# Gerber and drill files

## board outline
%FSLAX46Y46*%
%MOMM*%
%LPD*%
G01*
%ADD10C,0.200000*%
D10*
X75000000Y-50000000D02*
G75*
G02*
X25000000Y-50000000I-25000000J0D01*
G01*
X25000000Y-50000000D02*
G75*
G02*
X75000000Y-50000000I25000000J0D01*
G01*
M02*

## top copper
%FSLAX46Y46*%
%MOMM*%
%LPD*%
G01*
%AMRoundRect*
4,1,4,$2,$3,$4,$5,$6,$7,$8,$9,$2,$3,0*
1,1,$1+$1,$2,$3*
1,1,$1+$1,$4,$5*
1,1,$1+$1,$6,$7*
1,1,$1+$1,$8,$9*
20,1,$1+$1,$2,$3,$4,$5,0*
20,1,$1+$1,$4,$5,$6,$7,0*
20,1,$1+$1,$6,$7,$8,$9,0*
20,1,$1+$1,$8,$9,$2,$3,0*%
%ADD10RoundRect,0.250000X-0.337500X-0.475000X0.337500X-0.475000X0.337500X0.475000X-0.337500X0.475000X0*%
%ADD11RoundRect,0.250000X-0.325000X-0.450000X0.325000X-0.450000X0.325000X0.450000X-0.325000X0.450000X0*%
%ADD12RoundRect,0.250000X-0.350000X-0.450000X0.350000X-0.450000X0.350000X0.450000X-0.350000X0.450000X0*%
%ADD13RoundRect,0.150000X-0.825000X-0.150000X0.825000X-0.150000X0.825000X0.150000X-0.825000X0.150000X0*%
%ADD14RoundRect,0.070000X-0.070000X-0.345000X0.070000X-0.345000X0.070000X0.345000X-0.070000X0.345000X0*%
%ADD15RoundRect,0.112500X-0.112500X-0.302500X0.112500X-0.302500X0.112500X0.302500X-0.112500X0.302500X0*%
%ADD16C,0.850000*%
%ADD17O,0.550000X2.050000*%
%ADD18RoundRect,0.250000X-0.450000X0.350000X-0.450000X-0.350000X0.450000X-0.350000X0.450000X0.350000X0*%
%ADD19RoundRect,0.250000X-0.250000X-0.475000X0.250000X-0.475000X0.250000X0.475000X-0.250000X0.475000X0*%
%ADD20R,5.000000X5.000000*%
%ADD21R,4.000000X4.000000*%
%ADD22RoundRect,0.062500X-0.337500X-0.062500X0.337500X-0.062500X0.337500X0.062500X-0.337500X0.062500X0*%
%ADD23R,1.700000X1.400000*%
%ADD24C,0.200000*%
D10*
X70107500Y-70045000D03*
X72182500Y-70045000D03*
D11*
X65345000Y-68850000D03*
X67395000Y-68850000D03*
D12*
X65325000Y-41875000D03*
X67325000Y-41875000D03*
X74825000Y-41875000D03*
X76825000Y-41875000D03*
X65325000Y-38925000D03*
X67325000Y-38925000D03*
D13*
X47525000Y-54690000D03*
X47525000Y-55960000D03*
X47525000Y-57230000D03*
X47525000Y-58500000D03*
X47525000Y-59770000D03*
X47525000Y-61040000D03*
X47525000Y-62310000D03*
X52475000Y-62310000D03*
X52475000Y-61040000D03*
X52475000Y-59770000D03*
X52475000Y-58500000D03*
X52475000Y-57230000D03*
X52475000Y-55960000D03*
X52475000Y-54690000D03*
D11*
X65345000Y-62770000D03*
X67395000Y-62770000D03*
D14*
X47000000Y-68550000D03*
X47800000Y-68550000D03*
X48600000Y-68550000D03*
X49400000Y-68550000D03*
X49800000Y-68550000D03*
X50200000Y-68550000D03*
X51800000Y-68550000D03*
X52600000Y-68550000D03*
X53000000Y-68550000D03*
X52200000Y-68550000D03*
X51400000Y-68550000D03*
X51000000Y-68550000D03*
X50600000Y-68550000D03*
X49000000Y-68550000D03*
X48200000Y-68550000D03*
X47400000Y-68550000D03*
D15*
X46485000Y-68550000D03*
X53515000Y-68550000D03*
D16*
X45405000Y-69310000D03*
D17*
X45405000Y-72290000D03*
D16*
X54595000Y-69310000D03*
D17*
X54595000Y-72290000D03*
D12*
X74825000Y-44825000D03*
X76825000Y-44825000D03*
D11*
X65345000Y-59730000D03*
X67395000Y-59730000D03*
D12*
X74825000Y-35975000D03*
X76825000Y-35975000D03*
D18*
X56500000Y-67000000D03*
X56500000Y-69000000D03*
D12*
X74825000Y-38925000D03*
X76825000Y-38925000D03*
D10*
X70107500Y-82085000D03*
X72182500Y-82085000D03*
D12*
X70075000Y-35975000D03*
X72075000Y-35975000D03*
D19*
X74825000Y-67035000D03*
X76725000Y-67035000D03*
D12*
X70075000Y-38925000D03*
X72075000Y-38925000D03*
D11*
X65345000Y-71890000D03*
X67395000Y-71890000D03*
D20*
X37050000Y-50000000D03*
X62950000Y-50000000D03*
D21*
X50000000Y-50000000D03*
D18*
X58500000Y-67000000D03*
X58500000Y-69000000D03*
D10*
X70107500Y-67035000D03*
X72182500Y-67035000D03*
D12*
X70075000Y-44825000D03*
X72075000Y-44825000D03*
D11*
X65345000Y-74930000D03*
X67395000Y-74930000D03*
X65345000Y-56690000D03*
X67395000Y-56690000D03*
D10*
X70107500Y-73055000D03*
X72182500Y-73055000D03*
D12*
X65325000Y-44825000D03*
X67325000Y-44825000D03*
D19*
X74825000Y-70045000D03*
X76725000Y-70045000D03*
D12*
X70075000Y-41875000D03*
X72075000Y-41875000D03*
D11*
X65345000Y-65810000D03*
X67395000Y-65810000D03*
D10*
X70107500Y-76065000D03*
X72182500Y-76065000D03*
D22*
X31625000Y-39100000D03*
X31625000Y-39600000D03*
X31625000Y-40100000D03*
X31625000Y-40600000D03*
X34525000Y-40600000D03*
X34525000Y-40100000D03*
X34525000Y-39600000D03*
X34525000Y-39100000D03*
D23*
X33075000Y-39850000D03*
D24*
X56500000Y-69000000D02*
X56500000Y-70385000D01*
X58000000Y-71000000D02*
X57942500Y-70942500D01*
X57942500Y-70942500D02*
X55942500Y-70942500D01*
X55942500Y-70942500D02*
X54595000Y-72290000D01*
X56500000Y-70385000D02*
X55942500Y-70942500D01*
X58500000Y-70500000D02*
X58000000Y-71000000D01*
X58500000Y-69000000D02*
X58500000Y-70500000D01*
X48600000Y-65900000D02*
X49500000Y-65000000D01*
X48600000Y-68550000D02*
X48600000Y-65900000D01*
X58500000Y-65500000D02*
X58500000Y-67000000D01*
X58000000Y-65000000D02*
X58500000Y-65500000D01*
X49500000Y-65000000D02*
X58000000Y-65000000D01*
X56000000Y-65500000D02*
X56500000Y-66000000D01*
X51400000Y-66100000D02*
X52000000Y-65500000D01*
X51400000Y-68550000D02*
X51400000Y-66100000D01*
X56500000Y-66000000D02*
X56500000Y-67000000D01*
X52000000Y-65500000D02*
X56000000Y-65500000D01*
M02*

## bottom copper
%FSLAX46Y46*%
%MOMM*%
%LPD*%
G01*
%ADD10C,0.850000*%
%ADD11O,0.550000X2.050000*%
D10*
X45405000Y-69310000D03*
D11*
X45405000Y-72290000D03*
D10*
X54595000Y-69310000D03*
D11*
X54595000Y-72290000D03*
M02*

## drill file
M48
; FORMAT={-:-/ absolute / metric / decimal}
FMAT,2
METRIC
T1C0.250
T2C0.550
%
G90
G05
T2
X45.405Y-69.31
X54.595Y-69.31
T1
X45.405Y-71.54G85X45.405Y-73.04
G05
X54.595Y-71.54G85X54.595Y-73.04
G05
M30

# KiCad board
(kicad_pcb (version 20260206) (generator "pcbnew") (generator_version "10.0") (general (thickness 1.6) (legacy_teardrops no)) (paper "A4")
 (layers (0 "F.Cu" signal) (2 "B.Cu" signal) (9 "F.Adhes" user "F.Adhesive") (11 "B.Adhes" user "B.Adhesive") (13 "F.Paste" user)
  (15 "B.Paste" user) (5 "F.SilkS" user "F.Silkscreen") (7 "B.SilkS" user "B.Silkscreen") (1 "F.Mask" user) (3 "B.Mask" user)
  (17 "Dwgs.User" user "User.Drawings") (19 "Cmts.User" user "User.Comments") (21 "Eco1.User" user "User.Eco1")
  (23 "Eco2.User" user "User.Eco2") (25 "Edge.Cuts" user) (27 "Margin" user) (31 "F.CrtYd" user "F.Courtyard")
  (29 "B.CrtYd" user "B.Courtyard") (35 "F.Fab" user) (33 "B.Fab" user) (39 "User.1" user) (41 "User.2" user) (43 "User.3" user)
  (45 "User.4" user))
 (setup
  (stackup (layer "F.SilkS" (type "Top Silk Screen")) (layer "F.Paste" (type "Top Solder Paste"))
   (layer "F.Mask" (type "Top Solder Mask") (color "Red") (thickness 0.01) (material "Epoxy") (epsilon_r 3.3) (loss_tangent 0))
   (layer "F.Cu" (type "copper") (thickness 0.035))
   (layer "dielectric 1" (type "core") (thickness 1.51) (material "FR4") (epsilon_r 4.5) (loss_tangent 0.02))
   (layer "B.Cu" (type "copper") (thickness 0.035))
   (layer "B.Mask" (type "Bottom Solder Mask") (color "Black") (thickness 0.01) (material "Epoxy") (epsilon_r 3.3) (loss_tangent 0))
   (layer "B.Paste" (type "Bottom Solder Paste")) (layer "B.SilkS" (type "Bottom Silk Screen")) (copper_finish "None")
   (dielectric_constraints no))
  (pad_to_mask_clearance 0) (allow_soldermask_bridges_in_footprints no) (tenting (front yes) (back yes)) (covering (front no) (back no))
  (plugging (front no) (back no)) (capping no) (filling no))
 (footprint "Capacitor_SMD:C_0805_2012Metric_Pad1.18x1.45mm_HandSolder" (layer "F.Cu") (at 71.145 70.045)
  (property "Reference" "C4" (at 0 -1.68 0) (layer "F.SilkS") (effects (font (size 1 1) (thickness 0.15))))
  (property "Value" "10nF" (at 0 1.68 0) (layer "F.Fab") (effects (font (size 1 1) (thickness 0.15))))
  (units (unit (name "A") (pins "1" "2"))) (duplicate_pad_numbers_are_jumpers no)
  (pad "1" smd roundrect (at -1.0375 0) (size 1.175 1.45) (layers "F.Cu" "F.Mask" "F.Paste") (roundrect_rratio 0.212766) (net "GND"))
  (pad "2" smd roundrect (at 1.0375 0) (size 1.175 1.45) (layers "F.Cu" "F.Mask" "F.Paste") (roundrect_rratio 0.212766)
   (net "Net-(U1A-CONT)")))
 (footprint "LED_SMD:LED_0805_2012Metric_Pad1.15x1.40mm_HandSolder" (layer "F.Cu") (at 66.37 68.85)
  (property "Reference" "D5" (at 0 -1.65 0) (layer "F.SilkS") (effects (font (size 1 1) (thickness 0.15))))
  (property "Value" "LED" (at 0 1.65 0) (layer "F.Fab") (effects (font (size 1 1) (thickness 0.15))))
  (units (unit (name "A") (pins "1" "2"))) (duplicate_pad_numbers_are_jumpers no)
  (pad "1" smd roundrect (at -1.025 0) (size 1.15 1.4) (layers "F.Cu" "F.Mask" "F.Paste") (roundrect_rratio 0.217391) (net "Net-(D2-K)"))
  (pad "2" smd roundrect (at 1.025 0) (size 1.15 1.4) (layers "F.Cu" "F.Mask" "F.Paste") (roundrect_rratio 0.217391) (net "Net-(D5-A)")))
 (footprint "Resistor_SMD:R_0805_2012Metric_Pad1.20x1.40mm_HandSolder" (layer "F.Cu") (at 66.325 41.875)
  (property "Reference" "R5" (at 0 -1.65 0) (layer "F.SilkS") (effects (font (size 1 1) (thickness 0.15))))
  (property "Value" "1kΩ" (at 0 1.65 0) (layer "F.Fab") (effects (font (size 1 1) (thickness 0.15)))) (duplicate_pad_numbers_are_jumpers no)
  (pad "1" smd roundrect (at -1 0) (size 1.2 1.4) (layers "F.Cu" "F.Mask" "F.Paste") (roundrect_rratio 0.208333) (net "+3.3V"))
  (pad "2" smd roundrect (at 1 0) (size 1.2 1.4) (layers "F.Cu" "F.Mask" "F.Paste") (roundrect_rratio 0.208333) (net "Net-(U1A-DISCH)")))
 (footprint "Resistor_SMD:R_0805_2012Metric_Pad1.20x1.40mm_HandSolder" (layer "F.Cu") (at 75.825 41.875)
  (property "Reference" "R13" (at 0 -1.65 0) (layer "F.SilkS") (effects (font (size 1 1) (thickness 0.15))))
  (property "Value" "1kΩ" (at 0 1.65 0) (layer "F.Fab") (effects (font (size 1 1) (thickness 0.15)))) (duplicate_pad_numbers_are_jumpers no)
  (pad "1" smd roundrect (at -1 0) (size 1.2 1.4) (layers "F.Cu" "F.Mask" "F.Paste") (roundrect_rratio 0.208333) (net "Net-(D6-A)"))
  (pad "2" smd roundrect (at 1 0) (size 1.2 1.4) (layers "F.Cu" "F.Mask" "F.Paste") (roundrect_rratio 0.208333) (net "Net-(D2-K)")))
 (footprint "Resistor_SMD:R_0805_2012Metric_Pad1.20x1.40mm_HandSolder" (layer "F.Cu") (at 66.325 38.925)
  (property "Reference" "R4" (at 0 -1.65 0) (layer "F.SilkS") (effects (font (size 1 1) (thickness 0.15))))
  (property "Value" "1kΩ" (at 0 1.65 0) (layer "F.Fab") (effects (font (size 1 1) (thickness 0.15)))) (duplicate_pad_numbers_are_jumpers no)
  (pad "1" smd roundrect (at -1 0) (size 1.2 1.4) (layers "F.Cu" "F.Mask" "F.Paste") (roundrect_rratio 0.208333) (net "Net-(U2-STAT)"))
  (pad "2" smd roundrect (at 1 0) (size 1.2 1.4) (layers "F.Cu" "F.Mask" "F.Paste") (roundrect_rratio 0.208333) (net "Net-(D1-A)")))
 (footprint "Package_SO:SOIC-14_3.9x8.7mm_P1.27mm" (layer "F.Cu") (at 50 58.5)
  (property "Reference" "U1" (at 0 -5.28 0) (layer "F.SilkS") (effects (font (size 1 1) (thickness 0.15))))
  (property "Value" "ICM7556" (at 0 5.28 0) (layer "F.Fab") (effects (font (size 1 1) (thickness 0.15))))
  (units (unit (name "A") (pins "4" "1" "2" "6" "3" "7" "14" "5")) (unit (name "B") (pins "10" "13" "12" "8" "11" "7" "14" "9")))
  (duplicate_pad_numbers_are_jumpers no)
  (pad "1" smd roundrect (at -2.475 -3.81) (size 1.95 0.6) (layers "F.Cu" "F.Mask" "F.Paste") (roundrect_rratio 0.25)
   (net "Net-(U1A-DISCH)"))
  (pad "2" smd roundrect (at -2.475 -2.54) (size 1.95 0.6) (layers "F.Cu" "F.Mask" "F.Paste") (roundrect_rratio 0.25)
   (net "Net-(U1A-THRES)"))
  (pad "3" smd roundrect (at -2.475 -1.27) (size 1.95 0.6) (layers "F.Cu" "F.Mask" "F.Paste") (roundrect_rratio 0.25) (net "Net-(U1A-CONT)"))
  (pad "4" smd roundrect (at -2.475 0) (size 1.95 0.6) (layers "F.Cu" "F.Mask" "F.Paste") (roundrect_rratio 0.25) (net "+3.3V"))
  (pad "5" smd roundrect (at -2.475 1.27) (size 1.95 0.6) (layers "F.Cu" "F.Mask" "F.Paste") (roundrect_rratio 0.25) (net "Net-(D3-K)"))
  (pad "6" smd roundrect (at -2.475 2.54) (size 1.95 0.6) (layers "F.Cu" "F.Mask" "F.Paste") (roundrect_rratio 0.25) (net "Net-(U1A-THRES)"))
  (pad "7" smd roundrect (at -2.475 3.81) (size 1.95 0.6) (layers "F.Cu" "F.Mask" "F.Paste") (roundrect_rratio 0.25) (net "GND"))
  (pad "8" smd roundrect (at 2.475 3.81) (size 1.95 0.6) (layers "F.Cu" "F.Mask" "F.Paste") (roundrect_rratio 0.25) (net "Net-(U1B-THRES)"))
  (pad "9" smd roundrect (at 2.475 2.54) (size 1.95 0.6) (layers "F.Cu" "F.Mask" "F.Paste") (roundrect_rratio 0.25) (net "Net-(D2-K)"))
  (pad "10" smd roundrect (at 2.475 1.27) (size 1.95 0.6) (layers "F.Cu" "F.Mask" "F.Paste") (roundrect_rratio 0.25) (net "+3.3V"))
  (pad "11" smd roundrect (at 2.475 0) (size 1.95 0.6) (layers "F.Cu" "F.Mask" "F.Paste") (roundrect_rratio 0.25) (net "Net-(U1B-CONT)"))
  (pad "12" smd roundrect (at 2.475 -1.27) (size 1.95 0.6) (layers "F.Cu" "F.Mask" "F.Paste") (roundrect_rratio 0.25)
   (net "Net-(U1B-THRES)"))
  (pad "13" smd roundrect (at 2.475 -2.54) (size 1.95 0.6) (layers "F.Cu" "F.Mask" "F.Paste") (roundrect_rratio 0.25)
   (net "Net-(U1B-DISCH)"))
  (pad "14" smd roundrect (at 2.475 -3.81) (size 1.95 0.6) (layers "F.Cu" "F.Mask" "F.Paste") (roundrect_rratio 0.25) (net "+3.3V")))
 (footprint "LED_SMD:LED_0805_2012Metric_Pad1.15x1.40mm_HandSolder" (layer "F.Cu") (at 66.37 62.77)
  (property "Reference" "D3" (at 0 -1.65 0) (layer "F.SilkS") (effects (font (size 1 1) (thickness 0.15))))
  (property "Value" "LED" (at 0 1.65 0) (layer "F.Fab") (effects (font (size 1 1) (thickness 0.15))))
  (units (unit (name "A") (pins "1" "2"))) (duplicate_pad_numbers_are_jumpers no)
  (pad "1" smd roundrect (at -1.025 0) (size 1.15 1.4) (layers "F.Cu" "F.Mask" "F.Paste") (roundrect_rratio 0.217391) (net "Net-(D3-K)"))
  (pad "2" smd roundrect (at 1.025 0) (size 1.15 1.4) (layers "F.Cu" "F.Mask" "F.Paste") (roundrect_rratio 0.217391) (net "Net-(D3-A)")))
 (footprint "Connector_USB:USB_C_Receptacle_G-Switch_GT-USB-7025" (layer "F.Cu") (at 50 72)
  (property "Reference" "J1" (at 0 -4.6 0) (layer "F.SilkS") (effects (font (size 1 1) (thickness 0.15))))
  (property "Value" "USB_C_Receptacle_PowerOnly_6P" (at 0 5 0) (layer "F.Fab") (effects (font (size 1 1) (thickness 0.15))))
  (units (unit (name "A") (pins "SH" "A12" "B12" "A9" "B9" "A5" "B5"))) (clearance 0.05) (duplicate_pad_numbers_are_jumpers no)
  (pad "A1" smd roundrect (at -3 -3.45) (size 0.28 0.83) (layers "F.Cu" "F.Mask" "F.Paste") (roundrect_rratio 0.25))
  (pad "A4" smd roundrect (at -2.2 -3.45) (size 0.28 0.83) (layers "F.Cu" "F.Mask" "F.Paste") (roundrect_rratio 0.25))
  (pad "A5" smd roundrect (at -1.4 -3.45) (size 0.28 0.83) (layers "F.Cu" "F.Mask" "F.Paste") (roundrect_rratio 0.25) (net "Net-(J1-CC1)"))
  (pad "A6" smd roundrect (at -0.6 -3.45) (size 0.28 0.83) (layers "F.Cu" "F.Mask" "F.Paste") (roundrect_rratio 0.25))
  (pad "A7" smd roundrect (at -0.2 -3.45) (size 0.28 0.83) (layers "F.Cu" "F.Mask" "F.Paste") (roundrect_rratio 0.25))
  (pad "A8" smd roundrect (at 0.2 -3.45) (size 0.28 0.83) (layers "F.Cu" "F.Mask" "F.Paste") (roundrect_rratio 0.25))
  (pad "A9" smd roundrect (at 1.8 -3.45) (size 0.28 0.83) (layers "F.Cu" "F.Mask" "F.Paste") (roundrect_rratio 0.25) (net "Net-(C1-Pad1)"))
  (pad "A12" smd roundrect (at 2.6 -3.45) (size 0.28 0.83) (layers "F.Cu" "F.Mask" "F.Paste") (roundrect_rratio 0.25) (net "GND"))
  (pad "B1" smd roundrect (at 3 -3.45) (size 0.28 0.83) (layers "F.Cu" "F.Mask" "F.Paste") (roundrect_rratio 0.25))
  (pad "B4" smd roundrect (at 2.2 -3.45) (size 0.28 0.83) (layers "F.Cu" "F.Mask" "F.Paste") (roundrect_rratio 0.25))
  (pad "B5" smd roundrect (at 1.4 -3.45) (size 0.28 0.83) (layers "F.Cu" "F.Mask" "F.Paste") (roundrect_rratio 0.25) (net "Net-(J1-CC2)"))
  (pad "B6" smd roundrect (at 1 -3.45) (size 0.28 0.83) (layers "F.Cu" "F.Mask" "F.Paste") (roundrect_rratio 0.25))
  (pad "B7" smd roundrect (at 0.6 -3.45) (size 0.28 0.83) (layers "F.Cu" "F.Mask" "F.Paste") (roundrect_rratio 0.25))
  (pad "B8" smd roundrect (at -1 -3.45) (size 0.28 0.83) (layers "F.Cu" "F.Mask" "F.Paste") (roundrect_rratio 0.25))
  (pad "B9" smd roundrect (at -1.8 -3.45) (size 0.28 0.83) (layers "F.Cu" "F.Mask" "F.Paste") (roundrect_rratio 0.25) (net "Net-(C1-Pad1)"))
  (pad "B12" smd roundrect (at -2.6 -3.45) (size 0.28 0.83) (layers "F.Cu" "F.Mask" "F.Paste") (roundrect_rratio 0.25) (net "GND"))
  (pad "GND" smd roundrect (at -3.515 -3.45) (size 0.45 0.83) (layers "F.Cu" "F.Mask" "F.Paste") (roundrect_rratio 0.25))
  (pad "GND" smd roundrect (at 3.515 -3.45) (size 0.45 0.83) (layers "F.Cu" "F.Mask" "F.Paste") (roundrect_rratio 0.25))
  (pad "SH" thru_hole circle (at -4.595 -2.69) (size 0.85 0.85) (drill 0.55) (layers "*.Cu" "*.Mask") (remove_unused_layers no) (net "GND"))
  (pad "SH" thru_hole oval (at -4.595 0.29) (size 0.55 2.05) (drill oval 0.25 1.75) (layers "*.Cu" "*.Mask") (remove_unused_layers no)
   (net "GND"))
  (pad "SH" thru_hole circle (at 4.595 -2.69) (size 0.85 0.85) (drill 0.55) (layers "*.Cu" "*.Mask") (remove_unused_layers no) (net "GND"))
  (pad "SH" thru_hole oval (at 4.595 0.29) (size 0.55 2.05) (drill oval 0.25 1.75) (layers "*.Cu" "*.Mask") (remove_unused_layers no)
   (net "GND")))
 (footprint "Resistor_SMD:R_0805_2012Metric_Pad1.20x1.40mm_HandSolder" (layer "F.Cu") (at 75.825 44.825)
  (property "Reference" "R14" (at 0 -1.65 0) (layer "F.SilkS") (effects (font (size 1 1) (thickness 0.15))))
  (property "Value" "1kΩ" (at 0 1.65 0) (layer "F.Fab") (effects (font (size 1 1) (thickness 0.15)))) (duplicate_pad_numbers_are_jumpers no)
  (pad "1" smd roundrect (at -1 0) (size 1.2 1.4) (layers "F.Cu" "F.Mask" "F.Paste") (roundrect_rratio 0.208333) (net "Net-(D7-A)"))
  (pad "2" smd roundrect (at 1 0) (size 1.2 1.4) (layers "F.Cu" "F.Mask" "F.Paste") (roundrect_rratio 0.208333) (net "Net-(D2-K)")))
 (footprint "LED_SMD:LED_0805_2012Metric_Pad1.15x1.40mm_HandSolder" (layer "F.Cu") (at 66.37 59.73)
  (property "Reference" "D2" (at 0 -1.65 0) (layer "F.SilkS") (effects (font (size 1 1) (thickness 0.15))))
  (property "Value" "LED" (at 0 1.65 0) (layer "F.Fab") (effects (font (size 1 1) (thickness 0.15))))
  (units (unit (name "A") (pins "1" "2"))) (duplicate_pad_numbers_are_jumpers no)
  (pad "1" smd roundrect (at -1.025 0) (size 1.15 1.4) (layers "F.Cu" "F.Mask" "F.Paste") (roundrect_rratio 0.217391) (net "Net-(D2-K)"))
  (pad "2" smd roundrect (at 1.025 0) (size 1.15 1.4) (layers "F.Cu" "F.Mask" "F.Paste") (roundrect_rratio 0.217391) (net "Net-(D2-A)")))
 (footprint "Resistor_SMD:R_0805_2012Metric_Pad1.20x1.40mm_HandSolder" (layer "F.Cu") (at 75.825 35.975)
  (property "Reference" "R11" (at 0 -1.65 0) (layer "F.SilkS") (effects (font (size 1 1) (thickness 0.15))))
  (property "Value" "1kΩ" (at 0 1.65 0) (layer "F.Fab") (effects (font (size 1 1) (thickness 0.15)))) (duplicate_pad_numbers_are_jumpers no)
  (pad "1" smd roundrect (at -1 0) (size 1.2 1.4) (layers "F.Cu" "F.Mask" "F.Paste") (roundrect_rratio 0.208333) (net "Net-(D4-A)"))
  (pad "2" smd roundrect (at 1 0) (size 1.2 1.4) (layers "F.Cu" "F.Mask" "F.Paste") (roundrect_rratio 0.208333) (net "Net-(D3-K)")))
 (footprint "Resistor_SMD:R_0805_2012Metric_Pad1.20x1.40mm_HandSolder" (layer "F.Cu") (at 56.5 68 -90)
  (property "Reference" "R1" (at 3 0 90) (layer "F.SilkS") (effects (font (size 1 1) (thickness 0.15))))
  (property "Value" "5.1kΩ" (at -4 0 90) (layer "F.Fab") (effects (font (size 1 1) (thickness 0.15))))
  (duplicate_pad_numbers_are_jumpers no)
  (pad "1" smd roundrect (at -1 0 270) (size 1.2 1.4) (layers "F.Cu" "F.Mask" "F.Paste") (roundrect_rratio 0.208333) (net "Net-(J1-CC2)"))
  (pad "2" smd roundrect (at 1 0 270) (size 1.2 1.4) (layers "F.Cu" "F.Mask" "F.Paste") (roundrect_rratio 0.208333) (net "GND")))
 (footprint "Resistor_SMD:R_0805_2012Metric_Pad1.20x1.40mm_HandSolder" (layer "F.Cu") (at 75.825 38.925)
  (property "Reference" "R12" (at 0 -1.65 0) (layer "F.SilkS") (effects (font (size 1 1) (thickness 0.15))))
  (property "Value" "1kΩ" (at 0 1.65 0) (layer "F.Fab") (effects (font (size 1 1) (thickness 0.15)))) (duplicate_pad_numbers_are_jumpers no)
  (pad "1" smd roundrect (at -1 0) (size 1.2 1.4) (layers "F.Cu" "F.Mask" "F.Paste") (roundrect_rratio 0.208333) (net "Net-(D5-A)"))
  (pad "2" smd roundrect (at 1 0) (size 1.2 1.4) (layers "F.Cu" "F.Mask" "F.Paste") (roundrect_rratio 0.208333) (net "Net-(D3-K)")))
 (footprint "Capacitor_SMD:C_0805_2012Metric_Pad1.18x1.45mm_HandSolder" (layer "F.Cu") (at 71.145 82.085)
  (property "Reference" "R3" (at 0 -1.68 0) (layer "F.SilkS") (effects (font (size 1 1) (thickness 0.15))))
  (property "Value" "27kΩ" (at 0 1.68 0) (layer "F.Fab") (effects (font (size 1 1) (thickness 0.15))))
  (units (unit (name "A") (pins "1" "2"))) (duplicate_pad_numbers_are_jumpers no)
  (pad "1" smd roundrect (at -1.0375 0) (size 1.175 1.45) (layers "F.Cu" "F.Mask" "F.Paste") (roundrect_rratio 0.212766)
   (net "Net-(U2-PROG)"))
  (pad "2" smd roundrect (at 1.0375 0) (size 1.175 1.45) (layers "F.Cu" "F.Mask" "F.Paste") (roundrect_rratio 0.212766) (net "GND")))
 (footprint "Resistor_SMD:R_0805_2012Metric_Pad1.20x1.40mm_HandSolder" (layer "F.Cu") (at 71.075 35.975)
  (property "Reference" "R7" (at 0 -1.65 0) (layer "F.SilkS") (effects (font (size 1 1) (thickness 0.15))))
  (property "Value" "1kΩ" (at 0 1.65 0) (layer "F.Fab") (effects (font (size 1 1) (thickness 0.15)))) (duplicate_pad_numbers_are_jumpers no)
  (pad "1" smd roundrect (at -1 0) (size 1.2 1.4) (layers "F.Cu" "F.Mask" "F.Paste") (roundrect_rratio 0.208333) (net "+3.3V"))
  (pad "2" smd roundrect (at 1 0) (size 1.2 1.4) (layers "F.Cu" "F.Mask" "F.Paste") (roundrect_rratio 0.208333) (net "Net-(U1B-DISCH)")))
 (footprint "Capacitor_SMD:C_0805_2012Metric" (layer "F.Cu") (at 75.775 67.035)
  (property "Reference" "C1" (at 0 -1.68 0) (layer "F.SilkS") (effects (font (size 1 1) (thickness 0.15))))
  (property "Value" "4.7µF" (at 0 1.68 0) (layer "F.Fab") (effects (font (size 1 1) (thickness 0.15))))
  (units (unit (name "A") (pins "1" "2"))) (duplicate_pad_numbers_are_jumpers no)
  (pad "1" smd roundrect (at -0.95 0) (size 1 1.45) (layers "F.Cu" "F.Mask" "F.Paste") (roundrect_rratio 0.25) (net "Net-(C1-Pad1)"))
  (pad "2" smd roundrect (at 0.95 0) (size 1 1.45) (layers "F.Cu" "F.Mask" "F.Paste") (roundrect_rratio 0.25) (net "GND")))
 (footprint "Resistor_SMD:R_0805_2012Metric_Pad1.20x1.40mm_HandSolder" (layer "F.Cu") (at 71.075 38.925)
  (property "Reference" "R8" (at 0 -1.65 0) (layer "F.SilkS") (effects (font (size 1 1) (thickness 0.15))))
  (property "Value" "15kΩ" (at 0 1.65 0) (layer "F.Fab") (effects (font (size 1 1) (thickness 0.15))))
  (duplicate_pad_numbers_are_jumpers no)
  (pad "1" smd roundrect (at -1 0) (size 1.2 1.4) (layers "F.Cu" "F.Mask" "F.Paste") (roundrect_rratio 0.208333) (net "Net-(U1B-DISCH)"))
  (pad "2" smd roundrect (at 1 0) (size 1.2 1.4) (layers "F.Cu" "F.Mask" "F.Paste") (roundrect_rratio 0.208333) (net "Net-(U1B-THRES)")))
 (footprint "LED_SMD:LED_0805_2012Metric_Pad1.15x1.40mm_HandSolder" (layer "F.Cu") (at 66.37 71.89)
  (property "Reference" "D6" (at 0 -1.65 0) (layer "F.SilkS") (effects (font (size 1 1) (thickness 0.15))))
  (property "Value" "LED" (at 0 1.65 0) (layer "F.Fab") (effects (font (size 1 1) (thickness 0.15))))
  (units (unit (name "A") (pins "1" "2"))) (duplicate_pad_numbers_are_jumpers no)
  (pad "1" smd roundrect (at -1.025 0) (size 1.15 1.4) (layers "F.Cu" "F.Mask" "F.Paste") (roundrect_rratio 0.217391) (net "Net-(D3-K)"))
  (pad "2" smd roundrect (at 1.025 0) (size 1.15 1.4) (layers "F.Cu" "F.Mask" "F.Paste") (roundrect_rratio 0.217391) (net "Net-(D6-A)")))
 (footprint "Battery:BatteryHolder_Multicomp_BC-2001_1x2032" (layer "F.Cu") (at 50 50)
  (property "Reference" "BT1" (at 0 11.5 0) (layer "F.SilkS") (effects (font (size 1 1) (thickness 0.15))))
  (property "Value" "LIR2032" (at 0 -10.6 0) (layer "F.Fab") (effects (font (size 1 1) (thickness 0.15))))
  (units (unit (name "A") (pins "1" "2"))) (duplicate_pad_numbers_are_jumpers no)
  (pad "1" smd rect (at -12.95 0) (size 5 5) (layers "F.Cu" "F.Mask" "F.Paste") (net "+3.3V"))
  (pad "1" smd rect (at 12.95 0) (size 5 5) (layers "F.Cu" "F.Mask" "F.Paste") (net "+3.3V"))
  (pad "2" smd rect (at 0 0) (size 4 4) (layers "F.Cu" "F.Mask" "F.Paste") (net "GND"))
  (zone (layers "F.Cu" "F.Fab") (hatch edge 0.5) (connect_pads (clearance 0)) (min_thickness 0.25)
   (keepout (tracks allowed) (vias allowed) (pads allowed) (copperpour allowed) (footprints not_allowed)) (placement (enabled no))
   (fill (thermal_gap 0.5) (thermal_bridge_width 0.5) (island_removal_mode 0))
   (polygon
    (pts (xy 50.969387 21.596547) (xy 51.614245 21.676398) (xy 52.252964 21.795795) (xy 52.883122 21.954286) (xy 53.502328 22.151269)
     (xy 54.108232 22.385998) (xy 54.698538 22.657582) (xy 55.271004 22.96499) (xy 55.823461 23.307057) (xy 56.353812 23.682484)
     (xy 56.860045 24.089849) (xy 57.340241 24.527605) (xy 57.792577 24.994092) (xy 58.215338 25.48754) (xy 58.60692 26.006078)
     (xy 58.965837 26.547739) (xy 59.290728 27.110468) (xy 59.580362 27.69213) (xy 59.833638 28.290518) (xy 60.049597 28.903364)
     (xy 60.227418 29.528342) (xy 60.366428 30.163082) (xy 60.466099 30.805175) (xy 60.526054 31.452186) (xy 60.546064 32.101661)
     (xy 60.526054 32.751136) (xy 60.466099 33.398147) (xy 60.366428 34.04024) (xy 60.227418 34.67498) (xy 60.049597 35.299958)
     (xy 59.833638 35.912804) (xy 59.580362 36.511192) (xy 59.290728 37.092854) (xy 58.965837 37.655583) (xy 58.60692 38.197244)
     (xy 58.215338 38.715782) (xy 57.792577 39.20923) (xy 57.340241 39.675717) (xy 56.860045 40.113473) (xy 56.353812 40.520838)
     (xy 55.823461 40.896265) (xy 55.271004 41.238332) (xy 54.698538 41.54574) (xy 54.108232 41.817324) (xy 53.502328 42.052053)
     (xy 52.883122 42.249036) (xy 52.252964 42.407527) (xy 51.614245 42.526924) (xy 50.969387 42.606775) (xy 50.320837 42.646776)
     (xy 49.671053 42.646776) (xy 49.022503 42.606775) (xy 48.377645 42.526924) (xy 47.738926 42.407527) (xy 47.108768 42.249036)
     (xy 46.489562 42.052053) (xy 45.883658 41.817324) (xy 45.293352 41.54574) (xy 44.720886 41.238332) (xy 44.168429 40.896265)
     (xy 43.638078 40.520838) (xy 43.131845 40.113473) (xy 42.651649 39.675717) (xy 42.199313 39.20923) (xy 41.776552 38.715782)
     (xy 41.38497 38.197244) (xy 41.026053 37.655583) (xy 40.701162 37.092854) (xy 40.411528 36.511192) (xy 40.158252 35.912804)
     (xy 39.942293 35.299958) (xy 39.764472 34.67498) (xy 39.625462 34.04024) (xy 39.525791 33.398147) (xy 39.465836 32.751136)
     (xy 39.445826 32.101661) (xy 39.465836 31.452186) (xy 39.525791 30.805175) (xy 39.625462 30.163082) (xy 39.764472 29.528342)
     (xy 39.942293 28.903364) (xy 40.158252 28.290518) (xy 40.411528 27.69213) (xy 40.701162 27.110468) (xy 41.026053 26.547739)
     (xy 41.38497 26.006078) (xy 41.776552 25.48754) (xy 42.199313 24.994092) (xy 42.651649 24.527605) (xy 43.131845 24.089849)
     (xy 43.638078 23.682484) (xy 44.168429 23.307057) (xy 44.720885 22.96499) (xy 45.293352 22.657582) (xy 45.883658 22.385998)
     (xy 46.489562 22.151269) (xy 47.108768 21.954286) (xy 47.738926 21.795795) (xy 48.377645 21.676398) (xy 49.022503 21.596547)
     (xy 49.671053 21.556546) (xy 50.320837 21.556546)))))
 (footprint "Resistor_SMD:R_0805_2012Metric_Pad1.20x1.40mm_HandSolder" (layer "F.Cu") (at 58.5 68 -90)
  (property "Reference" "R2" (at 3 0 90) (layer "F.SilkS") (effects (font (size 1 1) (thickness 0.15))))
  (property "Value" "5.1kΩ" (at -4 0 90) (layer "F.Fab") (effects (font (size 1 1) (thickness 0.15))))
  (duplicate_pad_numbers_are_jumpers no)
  (pad "1" smd roundrect (at -1 0 270) (size 1.2 1.4) (layers "F.Cu" "F.Mask" "F.Paste") (roundrect_rratio 0.208333) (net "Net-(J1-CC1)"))
  (pad "2" smd roundrect (at 1 0 270) (size 1.2 1.4) (layers "F.Cu" "F.Mask" "F.Paste") (roundrect_rratio 0.208333) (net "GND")))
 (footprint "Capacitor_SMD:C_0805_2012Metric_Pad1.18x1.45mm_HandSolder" (layer "F.Cu") (at 71.145 67.035)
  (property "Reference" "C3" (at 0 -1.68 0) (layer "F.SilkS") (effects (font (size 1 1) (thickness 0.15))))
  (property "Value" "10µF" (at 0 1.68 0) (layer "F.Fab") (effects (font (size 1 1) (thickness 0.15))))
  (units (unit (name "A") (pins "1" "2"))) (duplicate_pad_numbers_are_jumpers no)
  (pad "1" smd roundrect (at -1.0375 0) (size 1.175 1.45) (layers "F.Cu" "F.Mask" "F.Paste") (roundrect_rratio 0.212766)
   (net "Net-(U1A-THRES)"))
  (pad "2" smd roundrect (at 1.0375 0) (size 1.175 1.45) (layers "F.Cu" "F.Mask" "F.Paste") (roundrect_rratio 0.212766) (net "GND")))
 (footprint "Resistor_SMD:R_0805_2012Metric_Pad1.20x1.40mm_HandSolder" (layer "F.Cu") (at 71.075 44.825)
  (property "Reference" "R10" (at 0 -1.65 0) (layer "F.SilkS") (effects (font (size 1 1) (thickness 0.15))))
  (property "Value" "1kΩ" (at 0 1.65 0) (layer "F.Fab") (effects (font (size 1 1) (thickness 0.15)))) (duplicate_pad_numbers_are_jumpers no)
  (pad "1" smd roundrect (at -1 0) (size 1.2 1.4) (layers "F.Cu" "F.Mask" "F.Paste") (roundrect_rratio 0.208333) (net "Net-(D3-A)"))
  (pad "2" smd roundrect (at 1 0) (size 1.2 1.4) (layers "F.Cu" "F.Mask" "F.Paste") (roundrect_rratio 0.208333) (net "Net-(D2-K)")))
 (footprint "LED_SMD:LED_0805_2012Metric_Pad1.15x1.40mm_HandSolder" (layer "F.Cu") (at 66.37 74.93)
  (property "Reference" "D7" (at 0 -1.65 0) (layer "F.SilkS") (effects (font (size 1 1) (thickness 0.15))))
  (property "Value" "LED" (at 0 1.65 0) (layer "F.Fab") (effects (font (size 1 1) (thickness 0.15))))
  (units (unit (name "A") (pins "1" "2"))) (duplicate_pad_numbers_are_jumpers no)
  (pad "1" smd roundrect (at -1.025 0) (size 1.15 1.4) (layers "F.Cu" "F.Mask" "F.Paste") (roundrect_rratio 0.217391) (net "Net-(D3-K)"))
  (pad "2" smd roundrect (at 1.025 0) (size 1.15 1.4) (layers "F.Cu" "F.Mask" "F.Paste") (roundrect_rratio 0.217391) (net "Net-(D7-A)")))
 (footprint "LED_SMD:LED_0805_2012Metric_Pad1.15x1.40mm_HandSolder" (layer "F.Cu") (at 66.37 56.69)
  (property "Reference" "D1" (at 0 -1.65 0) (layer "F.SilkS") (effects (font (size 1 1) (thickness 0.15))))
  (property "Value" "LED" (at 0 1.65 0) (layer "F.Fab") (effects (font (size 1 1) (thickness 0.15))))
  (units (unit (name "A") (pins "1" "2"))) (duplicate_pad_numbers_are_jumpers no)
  (pad "1" smd roundrect (at -1.025 0) (size 1.15 1.4) (layers "F.Cu" "F.Mask" "F.Paste") (roundrect_rratio 0.217391) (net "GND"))
  (pad "2" smd roundrect (at 1.025 0) (size 1.15 1.4) (layers "F.Cu" "F.Mask" "F.Paste") (roundrect_rratio 0.217391) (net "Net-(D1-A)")))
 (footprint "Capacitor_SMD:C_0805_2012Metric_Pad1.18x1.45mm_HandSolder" (layer "F.Cu") (at 71.145 73.055)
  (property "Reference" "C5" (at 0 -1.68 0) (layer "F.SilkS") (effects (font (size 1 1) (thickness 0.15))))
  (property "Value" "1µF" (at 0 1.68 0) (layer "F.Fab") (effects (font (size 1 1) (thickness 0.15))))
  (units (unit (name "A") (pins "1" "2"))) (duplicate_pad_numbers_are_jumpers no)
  (pad "1" smd roundrect (at -1.0375 0) (size 1.175 1.45) (layers "F.Cu" "F.Mask" "F.Paste") (roundrect_rratio 0.212766)
   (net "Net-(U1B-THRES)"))
  (pad "2" smd roundrect (at 1.0375 0) (size 1.175 1.45) (layers "F.Cu" "F.Mask" "F.Paste") (roundrect_rratio 0.212766) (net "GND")))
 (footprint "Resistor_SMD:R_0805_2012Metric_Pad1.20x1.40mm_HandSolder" (layer "F.Cu") (at 66.325 44.825)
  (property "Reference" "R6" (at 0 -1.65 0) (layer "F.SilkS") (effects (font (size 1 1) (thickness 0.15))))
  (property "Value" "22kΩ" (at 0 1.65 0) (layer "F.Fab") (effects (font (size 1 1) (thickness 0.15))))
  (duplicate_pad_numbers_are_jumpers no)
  (pad "1" smd roundrect (at -1 0) (size 1.2 1.4) (layers "F.Cu" "F.Mask" "F.Paste") (roundrect_rratio 0.208333) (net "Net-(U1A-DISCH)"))
  (pad "2" smd roundrect (at 1 0) (size 1.2 1.4) (layers "F.Cu" "F.Mask" "F.Paste") (roundrect_rratio 0.208333) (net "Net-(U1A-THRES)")))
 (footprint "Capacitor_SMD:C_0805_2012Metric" (layer "F.Cu") (at 75.775 70.045)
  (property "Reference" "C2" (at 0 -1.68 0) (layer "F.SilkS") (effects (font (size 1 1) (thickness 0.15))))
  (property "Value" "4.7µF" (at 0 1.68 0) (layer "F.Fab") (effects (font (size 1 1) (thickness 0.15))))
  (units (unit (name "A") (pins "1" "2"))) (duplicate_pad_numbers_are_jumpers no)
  (pad "1" smd roundrect (at -0.95 0) (size 1 1.45) (layers "F.Cu" "F.Mask" "F.Paste") (roundrect_rratio 0.25) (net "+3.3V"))
  (pad "2" smd roundrect (at 0.95 0) (size 1 1.45) (layers "F.Cu" "F.Mask" "F.Paste") (roundrect_rratio 0.25) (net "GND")))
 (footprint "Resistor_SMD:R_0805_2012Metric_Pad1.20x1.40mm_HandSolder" (layer "F.Cu") (at 71.075 41.875)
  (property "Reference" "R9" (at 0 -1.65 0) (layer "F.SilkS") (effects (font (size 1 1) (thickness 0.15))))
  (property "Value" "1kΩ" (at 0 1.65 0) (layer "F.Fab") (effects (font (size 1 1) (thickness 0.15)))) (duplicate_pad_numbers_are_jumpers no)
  (pad "1" smd roundrect (at -1 0) (size 1.2 1.4) (layers "F.Cu" "F.Mask" "F.Paste") (roundrect_rratio 0.208333) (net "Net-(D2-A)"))
  (pad "2" smd roundrect (at 1 0) (size 1.2 1.4) (layers "F.Cu" "F.Mask" "F.Paste") (roundrect_rratio 0.208333) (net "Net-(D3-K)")))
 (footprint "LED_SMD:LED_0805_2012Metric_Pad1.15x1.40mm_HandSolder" (layer "F.Cu") (at 66.37 65.81)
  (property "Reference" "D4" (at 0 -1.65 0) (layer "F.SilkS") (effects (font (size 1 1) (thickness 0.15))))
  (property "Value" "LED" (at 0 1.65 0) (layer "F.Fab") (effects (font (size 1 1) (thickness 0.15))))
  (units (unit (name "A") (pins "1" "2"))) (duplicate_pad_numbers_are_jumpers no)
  (pad "1" smd roundrect (at -1.025 0) (size 1.15 1.4) (layers "F.Cu" "F.Mask" "F.Paste") (roundrect_rratio 0.217391) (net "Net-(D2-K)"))
  (pad "2" smd roundrect (at 1.025 0) (size 1.15 1.4) (layers "F.Cu" "F.Mask" "F.Paste") (roundrect_rratio 0.217391) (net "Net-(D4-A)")))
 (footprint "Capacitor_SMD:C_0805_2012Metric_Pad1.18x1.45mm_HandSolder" (layer "F.Cu") (at 71.145 76.065)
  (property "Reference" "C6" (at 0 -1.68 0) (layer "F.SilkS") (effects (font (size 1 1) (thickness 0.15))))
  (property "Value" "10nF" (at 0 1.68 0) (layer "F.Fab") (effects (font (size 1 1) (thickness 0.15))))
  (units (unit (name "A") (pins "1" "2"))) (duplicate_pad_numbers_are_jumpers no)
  (pad "1" smd roundrect (at -1.0375 0) (size 1.175 1.45) (layers "F.Cu" "F.Mask" "F.Paste") (roundrect_rratio 0.212766) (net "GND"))
  (pad "2" smd roundrect (at 1.0375 0) (size 1.175 1.45) (layers "F.Cu" "F.Mask" "F.Paste") (roundrect_rratio 0.212766)
   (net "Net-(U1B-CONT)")))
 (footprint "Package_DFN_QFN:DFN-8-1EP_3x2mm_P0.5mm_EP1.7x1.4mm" (layer "F.Cu") (at 33.075 39.85)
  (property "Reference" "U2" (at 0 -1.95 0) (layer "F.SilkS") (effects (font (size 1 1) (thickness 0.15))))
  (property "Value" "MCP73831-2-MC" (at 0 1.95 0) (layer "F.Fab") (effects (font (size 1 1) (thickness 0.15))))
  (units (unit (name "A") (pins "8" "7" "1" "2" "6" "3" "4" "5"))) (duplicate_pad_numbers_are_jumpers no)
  (pad "" smd roundrect (at -0.425 -0.35) (size 0.69 0.56) (layers "F.Paste") (roundrect_rratio 0.25))
  (pad "" smd roundrect (at -0.425 0.35) (size 0.69 0.56) (layers "F.Paste") (roundrect_rratio 0.25))
  (pad "" smd roundrect (at 0.425 -0.35) (size 0.69 0.56) (layers "F.Paste") (roundrect_rratio 0.25))
  (pad "" smd roundrect (at 0.425 0.35) (size 0.69 0.56) (layers "F.Paste") (roundrect_rratio 0.25))
  (pad "1" smd roundrect (at -1.45 -0.75) (size 0.8 0.25) (layers "F.Cu" "F.Mask" "F.Paste") (roundrect_rratio 0.25) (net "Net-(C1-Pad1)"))
  (pad "2" smd roundrect (at -1.45 -0.25) (size 0.8 0.25) (layers "F.Cu" "F.Mask" "F.Paste") (roundrect_rratio 0.25) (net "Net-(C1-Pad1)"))
  (pad "3" smd roundrect (at -1.45 0.25) (size 0.8 0.25) (layers "F.Cu" "F.Mask" "F.Paste") (roundrect_rratio 0.25) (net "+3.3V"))
  (pad "4" smd roundrect (at -1.45 0.75) (size 0.8 0.25) (layers "F.Cu" "F.Mask" "F.Paste") (roundrect_rratio 0.25) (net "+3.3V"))
  (pad "5" smd roundrect (at 1.45 0.75) (size 0.8 0.25) (layers "F.Cu" "F.Mask" "F.Paste") (roundrect_rratio 0.25) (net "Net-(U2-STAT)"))
  (pad "6" smd roundrect (at 1.45 0.25) (size 0.8 0.25) (layers "F.Cu" "F.Mask" "F.Paste") (roundrect_rratio 0.25) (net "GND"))
  (pad "7" smd roundrect (at 1.45 -0.25) (size 0.8 0.25) (layers "F.Cu" "F.Mask" "F.Paste") (roundrect_rratio 0.25)
   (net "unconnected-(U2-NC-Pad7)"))
  (pad "8" smd roundrect (at 1.45 -0.75) (size 0.8 0.25) (layers "F.Cu" "F.Mask" "F.Paste") (roundrect_rratio 0.25) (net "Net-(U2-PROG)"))
  (pad "9" smd rect (at 0 0) (size 1.7 1.4) (layers "F.Cu" "F.Mask") (zone_connect 2)))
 (gr_circle (center 50 50) (end 75 50) (stroke (width 0.2) (type default)) (fill no) (layer "Edge.Cuts"))
 (segment (start 56.5 69) (end 56.5 70.385) (width 0.2) (layer "F.Cu") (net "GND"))
 (segment (start 58 71) (end 57.9425 70.9425) (width 0.2) (layer "F.Cu") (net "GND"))
 (segment (start 57.9425 70.9425) (end 55.9425 70.9425) (width 0.2) (layer "F.Cu") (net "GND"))
 (segment (start 55.9425 70.9425) (end 54.595 72.29) (width 0.2) (layer "F.Cu") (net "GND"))
 (segment (start 56.5 70.385) (end 55.9425 70.9425) (width 0.2) (layer "F.Cu") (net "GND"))
 (segment (start 58.5 70.5) (end 58 71) (width 0.2) (layer "F.Cu") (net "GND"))
 (segment (start 58.5 69) (end 58.5 70.5) (width 0.2) (layer "F.Cu") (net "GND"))
 (segment (start 48.6 65.9) (end 49.5 65) (width 0.2) (layer "F.Cu") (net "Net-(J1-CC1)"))
 (segment (start 48.6 68.55) (end 48.6 65.9) (width 0.2) (layer "F.Cu") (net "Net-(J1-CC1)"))
 (segment (start 58.5 65.5) (end 58.5 67) (width 0.2) (layer "F.Cu") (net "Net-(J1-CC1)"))
 (segment (start 58 65) (end 58.5 65.5) (width 0.2) (layer "F.Cu") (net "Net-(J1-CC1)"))
 (segment (start 49.5 65) (end 58 65) (width 0.2) (layer "F.Cu") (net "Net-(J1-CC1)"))
 (segment (start 56 65.5) (end 56.5 66) (width 0.2) (layer "F.Cu") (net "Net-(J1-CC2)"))
 (segment (start 51.4 66.1) (end 52 65.5) (width 0.2) (layer "F.Cu") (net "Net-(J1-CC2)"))
 (segment (start 51.4 68.55) (end 51.4 66.1) (width 0.2) (layer "F.Cu") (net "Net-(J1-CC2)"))
 (segment (start 56.5 66) (end 56.5 67) (width 0.2) (layer "F.Cu") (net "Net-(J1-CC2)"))
 (segment (start 52 65.5) (end 56 65.5) (width 0.2) (layer "F.Cu") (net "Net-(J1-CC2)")))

